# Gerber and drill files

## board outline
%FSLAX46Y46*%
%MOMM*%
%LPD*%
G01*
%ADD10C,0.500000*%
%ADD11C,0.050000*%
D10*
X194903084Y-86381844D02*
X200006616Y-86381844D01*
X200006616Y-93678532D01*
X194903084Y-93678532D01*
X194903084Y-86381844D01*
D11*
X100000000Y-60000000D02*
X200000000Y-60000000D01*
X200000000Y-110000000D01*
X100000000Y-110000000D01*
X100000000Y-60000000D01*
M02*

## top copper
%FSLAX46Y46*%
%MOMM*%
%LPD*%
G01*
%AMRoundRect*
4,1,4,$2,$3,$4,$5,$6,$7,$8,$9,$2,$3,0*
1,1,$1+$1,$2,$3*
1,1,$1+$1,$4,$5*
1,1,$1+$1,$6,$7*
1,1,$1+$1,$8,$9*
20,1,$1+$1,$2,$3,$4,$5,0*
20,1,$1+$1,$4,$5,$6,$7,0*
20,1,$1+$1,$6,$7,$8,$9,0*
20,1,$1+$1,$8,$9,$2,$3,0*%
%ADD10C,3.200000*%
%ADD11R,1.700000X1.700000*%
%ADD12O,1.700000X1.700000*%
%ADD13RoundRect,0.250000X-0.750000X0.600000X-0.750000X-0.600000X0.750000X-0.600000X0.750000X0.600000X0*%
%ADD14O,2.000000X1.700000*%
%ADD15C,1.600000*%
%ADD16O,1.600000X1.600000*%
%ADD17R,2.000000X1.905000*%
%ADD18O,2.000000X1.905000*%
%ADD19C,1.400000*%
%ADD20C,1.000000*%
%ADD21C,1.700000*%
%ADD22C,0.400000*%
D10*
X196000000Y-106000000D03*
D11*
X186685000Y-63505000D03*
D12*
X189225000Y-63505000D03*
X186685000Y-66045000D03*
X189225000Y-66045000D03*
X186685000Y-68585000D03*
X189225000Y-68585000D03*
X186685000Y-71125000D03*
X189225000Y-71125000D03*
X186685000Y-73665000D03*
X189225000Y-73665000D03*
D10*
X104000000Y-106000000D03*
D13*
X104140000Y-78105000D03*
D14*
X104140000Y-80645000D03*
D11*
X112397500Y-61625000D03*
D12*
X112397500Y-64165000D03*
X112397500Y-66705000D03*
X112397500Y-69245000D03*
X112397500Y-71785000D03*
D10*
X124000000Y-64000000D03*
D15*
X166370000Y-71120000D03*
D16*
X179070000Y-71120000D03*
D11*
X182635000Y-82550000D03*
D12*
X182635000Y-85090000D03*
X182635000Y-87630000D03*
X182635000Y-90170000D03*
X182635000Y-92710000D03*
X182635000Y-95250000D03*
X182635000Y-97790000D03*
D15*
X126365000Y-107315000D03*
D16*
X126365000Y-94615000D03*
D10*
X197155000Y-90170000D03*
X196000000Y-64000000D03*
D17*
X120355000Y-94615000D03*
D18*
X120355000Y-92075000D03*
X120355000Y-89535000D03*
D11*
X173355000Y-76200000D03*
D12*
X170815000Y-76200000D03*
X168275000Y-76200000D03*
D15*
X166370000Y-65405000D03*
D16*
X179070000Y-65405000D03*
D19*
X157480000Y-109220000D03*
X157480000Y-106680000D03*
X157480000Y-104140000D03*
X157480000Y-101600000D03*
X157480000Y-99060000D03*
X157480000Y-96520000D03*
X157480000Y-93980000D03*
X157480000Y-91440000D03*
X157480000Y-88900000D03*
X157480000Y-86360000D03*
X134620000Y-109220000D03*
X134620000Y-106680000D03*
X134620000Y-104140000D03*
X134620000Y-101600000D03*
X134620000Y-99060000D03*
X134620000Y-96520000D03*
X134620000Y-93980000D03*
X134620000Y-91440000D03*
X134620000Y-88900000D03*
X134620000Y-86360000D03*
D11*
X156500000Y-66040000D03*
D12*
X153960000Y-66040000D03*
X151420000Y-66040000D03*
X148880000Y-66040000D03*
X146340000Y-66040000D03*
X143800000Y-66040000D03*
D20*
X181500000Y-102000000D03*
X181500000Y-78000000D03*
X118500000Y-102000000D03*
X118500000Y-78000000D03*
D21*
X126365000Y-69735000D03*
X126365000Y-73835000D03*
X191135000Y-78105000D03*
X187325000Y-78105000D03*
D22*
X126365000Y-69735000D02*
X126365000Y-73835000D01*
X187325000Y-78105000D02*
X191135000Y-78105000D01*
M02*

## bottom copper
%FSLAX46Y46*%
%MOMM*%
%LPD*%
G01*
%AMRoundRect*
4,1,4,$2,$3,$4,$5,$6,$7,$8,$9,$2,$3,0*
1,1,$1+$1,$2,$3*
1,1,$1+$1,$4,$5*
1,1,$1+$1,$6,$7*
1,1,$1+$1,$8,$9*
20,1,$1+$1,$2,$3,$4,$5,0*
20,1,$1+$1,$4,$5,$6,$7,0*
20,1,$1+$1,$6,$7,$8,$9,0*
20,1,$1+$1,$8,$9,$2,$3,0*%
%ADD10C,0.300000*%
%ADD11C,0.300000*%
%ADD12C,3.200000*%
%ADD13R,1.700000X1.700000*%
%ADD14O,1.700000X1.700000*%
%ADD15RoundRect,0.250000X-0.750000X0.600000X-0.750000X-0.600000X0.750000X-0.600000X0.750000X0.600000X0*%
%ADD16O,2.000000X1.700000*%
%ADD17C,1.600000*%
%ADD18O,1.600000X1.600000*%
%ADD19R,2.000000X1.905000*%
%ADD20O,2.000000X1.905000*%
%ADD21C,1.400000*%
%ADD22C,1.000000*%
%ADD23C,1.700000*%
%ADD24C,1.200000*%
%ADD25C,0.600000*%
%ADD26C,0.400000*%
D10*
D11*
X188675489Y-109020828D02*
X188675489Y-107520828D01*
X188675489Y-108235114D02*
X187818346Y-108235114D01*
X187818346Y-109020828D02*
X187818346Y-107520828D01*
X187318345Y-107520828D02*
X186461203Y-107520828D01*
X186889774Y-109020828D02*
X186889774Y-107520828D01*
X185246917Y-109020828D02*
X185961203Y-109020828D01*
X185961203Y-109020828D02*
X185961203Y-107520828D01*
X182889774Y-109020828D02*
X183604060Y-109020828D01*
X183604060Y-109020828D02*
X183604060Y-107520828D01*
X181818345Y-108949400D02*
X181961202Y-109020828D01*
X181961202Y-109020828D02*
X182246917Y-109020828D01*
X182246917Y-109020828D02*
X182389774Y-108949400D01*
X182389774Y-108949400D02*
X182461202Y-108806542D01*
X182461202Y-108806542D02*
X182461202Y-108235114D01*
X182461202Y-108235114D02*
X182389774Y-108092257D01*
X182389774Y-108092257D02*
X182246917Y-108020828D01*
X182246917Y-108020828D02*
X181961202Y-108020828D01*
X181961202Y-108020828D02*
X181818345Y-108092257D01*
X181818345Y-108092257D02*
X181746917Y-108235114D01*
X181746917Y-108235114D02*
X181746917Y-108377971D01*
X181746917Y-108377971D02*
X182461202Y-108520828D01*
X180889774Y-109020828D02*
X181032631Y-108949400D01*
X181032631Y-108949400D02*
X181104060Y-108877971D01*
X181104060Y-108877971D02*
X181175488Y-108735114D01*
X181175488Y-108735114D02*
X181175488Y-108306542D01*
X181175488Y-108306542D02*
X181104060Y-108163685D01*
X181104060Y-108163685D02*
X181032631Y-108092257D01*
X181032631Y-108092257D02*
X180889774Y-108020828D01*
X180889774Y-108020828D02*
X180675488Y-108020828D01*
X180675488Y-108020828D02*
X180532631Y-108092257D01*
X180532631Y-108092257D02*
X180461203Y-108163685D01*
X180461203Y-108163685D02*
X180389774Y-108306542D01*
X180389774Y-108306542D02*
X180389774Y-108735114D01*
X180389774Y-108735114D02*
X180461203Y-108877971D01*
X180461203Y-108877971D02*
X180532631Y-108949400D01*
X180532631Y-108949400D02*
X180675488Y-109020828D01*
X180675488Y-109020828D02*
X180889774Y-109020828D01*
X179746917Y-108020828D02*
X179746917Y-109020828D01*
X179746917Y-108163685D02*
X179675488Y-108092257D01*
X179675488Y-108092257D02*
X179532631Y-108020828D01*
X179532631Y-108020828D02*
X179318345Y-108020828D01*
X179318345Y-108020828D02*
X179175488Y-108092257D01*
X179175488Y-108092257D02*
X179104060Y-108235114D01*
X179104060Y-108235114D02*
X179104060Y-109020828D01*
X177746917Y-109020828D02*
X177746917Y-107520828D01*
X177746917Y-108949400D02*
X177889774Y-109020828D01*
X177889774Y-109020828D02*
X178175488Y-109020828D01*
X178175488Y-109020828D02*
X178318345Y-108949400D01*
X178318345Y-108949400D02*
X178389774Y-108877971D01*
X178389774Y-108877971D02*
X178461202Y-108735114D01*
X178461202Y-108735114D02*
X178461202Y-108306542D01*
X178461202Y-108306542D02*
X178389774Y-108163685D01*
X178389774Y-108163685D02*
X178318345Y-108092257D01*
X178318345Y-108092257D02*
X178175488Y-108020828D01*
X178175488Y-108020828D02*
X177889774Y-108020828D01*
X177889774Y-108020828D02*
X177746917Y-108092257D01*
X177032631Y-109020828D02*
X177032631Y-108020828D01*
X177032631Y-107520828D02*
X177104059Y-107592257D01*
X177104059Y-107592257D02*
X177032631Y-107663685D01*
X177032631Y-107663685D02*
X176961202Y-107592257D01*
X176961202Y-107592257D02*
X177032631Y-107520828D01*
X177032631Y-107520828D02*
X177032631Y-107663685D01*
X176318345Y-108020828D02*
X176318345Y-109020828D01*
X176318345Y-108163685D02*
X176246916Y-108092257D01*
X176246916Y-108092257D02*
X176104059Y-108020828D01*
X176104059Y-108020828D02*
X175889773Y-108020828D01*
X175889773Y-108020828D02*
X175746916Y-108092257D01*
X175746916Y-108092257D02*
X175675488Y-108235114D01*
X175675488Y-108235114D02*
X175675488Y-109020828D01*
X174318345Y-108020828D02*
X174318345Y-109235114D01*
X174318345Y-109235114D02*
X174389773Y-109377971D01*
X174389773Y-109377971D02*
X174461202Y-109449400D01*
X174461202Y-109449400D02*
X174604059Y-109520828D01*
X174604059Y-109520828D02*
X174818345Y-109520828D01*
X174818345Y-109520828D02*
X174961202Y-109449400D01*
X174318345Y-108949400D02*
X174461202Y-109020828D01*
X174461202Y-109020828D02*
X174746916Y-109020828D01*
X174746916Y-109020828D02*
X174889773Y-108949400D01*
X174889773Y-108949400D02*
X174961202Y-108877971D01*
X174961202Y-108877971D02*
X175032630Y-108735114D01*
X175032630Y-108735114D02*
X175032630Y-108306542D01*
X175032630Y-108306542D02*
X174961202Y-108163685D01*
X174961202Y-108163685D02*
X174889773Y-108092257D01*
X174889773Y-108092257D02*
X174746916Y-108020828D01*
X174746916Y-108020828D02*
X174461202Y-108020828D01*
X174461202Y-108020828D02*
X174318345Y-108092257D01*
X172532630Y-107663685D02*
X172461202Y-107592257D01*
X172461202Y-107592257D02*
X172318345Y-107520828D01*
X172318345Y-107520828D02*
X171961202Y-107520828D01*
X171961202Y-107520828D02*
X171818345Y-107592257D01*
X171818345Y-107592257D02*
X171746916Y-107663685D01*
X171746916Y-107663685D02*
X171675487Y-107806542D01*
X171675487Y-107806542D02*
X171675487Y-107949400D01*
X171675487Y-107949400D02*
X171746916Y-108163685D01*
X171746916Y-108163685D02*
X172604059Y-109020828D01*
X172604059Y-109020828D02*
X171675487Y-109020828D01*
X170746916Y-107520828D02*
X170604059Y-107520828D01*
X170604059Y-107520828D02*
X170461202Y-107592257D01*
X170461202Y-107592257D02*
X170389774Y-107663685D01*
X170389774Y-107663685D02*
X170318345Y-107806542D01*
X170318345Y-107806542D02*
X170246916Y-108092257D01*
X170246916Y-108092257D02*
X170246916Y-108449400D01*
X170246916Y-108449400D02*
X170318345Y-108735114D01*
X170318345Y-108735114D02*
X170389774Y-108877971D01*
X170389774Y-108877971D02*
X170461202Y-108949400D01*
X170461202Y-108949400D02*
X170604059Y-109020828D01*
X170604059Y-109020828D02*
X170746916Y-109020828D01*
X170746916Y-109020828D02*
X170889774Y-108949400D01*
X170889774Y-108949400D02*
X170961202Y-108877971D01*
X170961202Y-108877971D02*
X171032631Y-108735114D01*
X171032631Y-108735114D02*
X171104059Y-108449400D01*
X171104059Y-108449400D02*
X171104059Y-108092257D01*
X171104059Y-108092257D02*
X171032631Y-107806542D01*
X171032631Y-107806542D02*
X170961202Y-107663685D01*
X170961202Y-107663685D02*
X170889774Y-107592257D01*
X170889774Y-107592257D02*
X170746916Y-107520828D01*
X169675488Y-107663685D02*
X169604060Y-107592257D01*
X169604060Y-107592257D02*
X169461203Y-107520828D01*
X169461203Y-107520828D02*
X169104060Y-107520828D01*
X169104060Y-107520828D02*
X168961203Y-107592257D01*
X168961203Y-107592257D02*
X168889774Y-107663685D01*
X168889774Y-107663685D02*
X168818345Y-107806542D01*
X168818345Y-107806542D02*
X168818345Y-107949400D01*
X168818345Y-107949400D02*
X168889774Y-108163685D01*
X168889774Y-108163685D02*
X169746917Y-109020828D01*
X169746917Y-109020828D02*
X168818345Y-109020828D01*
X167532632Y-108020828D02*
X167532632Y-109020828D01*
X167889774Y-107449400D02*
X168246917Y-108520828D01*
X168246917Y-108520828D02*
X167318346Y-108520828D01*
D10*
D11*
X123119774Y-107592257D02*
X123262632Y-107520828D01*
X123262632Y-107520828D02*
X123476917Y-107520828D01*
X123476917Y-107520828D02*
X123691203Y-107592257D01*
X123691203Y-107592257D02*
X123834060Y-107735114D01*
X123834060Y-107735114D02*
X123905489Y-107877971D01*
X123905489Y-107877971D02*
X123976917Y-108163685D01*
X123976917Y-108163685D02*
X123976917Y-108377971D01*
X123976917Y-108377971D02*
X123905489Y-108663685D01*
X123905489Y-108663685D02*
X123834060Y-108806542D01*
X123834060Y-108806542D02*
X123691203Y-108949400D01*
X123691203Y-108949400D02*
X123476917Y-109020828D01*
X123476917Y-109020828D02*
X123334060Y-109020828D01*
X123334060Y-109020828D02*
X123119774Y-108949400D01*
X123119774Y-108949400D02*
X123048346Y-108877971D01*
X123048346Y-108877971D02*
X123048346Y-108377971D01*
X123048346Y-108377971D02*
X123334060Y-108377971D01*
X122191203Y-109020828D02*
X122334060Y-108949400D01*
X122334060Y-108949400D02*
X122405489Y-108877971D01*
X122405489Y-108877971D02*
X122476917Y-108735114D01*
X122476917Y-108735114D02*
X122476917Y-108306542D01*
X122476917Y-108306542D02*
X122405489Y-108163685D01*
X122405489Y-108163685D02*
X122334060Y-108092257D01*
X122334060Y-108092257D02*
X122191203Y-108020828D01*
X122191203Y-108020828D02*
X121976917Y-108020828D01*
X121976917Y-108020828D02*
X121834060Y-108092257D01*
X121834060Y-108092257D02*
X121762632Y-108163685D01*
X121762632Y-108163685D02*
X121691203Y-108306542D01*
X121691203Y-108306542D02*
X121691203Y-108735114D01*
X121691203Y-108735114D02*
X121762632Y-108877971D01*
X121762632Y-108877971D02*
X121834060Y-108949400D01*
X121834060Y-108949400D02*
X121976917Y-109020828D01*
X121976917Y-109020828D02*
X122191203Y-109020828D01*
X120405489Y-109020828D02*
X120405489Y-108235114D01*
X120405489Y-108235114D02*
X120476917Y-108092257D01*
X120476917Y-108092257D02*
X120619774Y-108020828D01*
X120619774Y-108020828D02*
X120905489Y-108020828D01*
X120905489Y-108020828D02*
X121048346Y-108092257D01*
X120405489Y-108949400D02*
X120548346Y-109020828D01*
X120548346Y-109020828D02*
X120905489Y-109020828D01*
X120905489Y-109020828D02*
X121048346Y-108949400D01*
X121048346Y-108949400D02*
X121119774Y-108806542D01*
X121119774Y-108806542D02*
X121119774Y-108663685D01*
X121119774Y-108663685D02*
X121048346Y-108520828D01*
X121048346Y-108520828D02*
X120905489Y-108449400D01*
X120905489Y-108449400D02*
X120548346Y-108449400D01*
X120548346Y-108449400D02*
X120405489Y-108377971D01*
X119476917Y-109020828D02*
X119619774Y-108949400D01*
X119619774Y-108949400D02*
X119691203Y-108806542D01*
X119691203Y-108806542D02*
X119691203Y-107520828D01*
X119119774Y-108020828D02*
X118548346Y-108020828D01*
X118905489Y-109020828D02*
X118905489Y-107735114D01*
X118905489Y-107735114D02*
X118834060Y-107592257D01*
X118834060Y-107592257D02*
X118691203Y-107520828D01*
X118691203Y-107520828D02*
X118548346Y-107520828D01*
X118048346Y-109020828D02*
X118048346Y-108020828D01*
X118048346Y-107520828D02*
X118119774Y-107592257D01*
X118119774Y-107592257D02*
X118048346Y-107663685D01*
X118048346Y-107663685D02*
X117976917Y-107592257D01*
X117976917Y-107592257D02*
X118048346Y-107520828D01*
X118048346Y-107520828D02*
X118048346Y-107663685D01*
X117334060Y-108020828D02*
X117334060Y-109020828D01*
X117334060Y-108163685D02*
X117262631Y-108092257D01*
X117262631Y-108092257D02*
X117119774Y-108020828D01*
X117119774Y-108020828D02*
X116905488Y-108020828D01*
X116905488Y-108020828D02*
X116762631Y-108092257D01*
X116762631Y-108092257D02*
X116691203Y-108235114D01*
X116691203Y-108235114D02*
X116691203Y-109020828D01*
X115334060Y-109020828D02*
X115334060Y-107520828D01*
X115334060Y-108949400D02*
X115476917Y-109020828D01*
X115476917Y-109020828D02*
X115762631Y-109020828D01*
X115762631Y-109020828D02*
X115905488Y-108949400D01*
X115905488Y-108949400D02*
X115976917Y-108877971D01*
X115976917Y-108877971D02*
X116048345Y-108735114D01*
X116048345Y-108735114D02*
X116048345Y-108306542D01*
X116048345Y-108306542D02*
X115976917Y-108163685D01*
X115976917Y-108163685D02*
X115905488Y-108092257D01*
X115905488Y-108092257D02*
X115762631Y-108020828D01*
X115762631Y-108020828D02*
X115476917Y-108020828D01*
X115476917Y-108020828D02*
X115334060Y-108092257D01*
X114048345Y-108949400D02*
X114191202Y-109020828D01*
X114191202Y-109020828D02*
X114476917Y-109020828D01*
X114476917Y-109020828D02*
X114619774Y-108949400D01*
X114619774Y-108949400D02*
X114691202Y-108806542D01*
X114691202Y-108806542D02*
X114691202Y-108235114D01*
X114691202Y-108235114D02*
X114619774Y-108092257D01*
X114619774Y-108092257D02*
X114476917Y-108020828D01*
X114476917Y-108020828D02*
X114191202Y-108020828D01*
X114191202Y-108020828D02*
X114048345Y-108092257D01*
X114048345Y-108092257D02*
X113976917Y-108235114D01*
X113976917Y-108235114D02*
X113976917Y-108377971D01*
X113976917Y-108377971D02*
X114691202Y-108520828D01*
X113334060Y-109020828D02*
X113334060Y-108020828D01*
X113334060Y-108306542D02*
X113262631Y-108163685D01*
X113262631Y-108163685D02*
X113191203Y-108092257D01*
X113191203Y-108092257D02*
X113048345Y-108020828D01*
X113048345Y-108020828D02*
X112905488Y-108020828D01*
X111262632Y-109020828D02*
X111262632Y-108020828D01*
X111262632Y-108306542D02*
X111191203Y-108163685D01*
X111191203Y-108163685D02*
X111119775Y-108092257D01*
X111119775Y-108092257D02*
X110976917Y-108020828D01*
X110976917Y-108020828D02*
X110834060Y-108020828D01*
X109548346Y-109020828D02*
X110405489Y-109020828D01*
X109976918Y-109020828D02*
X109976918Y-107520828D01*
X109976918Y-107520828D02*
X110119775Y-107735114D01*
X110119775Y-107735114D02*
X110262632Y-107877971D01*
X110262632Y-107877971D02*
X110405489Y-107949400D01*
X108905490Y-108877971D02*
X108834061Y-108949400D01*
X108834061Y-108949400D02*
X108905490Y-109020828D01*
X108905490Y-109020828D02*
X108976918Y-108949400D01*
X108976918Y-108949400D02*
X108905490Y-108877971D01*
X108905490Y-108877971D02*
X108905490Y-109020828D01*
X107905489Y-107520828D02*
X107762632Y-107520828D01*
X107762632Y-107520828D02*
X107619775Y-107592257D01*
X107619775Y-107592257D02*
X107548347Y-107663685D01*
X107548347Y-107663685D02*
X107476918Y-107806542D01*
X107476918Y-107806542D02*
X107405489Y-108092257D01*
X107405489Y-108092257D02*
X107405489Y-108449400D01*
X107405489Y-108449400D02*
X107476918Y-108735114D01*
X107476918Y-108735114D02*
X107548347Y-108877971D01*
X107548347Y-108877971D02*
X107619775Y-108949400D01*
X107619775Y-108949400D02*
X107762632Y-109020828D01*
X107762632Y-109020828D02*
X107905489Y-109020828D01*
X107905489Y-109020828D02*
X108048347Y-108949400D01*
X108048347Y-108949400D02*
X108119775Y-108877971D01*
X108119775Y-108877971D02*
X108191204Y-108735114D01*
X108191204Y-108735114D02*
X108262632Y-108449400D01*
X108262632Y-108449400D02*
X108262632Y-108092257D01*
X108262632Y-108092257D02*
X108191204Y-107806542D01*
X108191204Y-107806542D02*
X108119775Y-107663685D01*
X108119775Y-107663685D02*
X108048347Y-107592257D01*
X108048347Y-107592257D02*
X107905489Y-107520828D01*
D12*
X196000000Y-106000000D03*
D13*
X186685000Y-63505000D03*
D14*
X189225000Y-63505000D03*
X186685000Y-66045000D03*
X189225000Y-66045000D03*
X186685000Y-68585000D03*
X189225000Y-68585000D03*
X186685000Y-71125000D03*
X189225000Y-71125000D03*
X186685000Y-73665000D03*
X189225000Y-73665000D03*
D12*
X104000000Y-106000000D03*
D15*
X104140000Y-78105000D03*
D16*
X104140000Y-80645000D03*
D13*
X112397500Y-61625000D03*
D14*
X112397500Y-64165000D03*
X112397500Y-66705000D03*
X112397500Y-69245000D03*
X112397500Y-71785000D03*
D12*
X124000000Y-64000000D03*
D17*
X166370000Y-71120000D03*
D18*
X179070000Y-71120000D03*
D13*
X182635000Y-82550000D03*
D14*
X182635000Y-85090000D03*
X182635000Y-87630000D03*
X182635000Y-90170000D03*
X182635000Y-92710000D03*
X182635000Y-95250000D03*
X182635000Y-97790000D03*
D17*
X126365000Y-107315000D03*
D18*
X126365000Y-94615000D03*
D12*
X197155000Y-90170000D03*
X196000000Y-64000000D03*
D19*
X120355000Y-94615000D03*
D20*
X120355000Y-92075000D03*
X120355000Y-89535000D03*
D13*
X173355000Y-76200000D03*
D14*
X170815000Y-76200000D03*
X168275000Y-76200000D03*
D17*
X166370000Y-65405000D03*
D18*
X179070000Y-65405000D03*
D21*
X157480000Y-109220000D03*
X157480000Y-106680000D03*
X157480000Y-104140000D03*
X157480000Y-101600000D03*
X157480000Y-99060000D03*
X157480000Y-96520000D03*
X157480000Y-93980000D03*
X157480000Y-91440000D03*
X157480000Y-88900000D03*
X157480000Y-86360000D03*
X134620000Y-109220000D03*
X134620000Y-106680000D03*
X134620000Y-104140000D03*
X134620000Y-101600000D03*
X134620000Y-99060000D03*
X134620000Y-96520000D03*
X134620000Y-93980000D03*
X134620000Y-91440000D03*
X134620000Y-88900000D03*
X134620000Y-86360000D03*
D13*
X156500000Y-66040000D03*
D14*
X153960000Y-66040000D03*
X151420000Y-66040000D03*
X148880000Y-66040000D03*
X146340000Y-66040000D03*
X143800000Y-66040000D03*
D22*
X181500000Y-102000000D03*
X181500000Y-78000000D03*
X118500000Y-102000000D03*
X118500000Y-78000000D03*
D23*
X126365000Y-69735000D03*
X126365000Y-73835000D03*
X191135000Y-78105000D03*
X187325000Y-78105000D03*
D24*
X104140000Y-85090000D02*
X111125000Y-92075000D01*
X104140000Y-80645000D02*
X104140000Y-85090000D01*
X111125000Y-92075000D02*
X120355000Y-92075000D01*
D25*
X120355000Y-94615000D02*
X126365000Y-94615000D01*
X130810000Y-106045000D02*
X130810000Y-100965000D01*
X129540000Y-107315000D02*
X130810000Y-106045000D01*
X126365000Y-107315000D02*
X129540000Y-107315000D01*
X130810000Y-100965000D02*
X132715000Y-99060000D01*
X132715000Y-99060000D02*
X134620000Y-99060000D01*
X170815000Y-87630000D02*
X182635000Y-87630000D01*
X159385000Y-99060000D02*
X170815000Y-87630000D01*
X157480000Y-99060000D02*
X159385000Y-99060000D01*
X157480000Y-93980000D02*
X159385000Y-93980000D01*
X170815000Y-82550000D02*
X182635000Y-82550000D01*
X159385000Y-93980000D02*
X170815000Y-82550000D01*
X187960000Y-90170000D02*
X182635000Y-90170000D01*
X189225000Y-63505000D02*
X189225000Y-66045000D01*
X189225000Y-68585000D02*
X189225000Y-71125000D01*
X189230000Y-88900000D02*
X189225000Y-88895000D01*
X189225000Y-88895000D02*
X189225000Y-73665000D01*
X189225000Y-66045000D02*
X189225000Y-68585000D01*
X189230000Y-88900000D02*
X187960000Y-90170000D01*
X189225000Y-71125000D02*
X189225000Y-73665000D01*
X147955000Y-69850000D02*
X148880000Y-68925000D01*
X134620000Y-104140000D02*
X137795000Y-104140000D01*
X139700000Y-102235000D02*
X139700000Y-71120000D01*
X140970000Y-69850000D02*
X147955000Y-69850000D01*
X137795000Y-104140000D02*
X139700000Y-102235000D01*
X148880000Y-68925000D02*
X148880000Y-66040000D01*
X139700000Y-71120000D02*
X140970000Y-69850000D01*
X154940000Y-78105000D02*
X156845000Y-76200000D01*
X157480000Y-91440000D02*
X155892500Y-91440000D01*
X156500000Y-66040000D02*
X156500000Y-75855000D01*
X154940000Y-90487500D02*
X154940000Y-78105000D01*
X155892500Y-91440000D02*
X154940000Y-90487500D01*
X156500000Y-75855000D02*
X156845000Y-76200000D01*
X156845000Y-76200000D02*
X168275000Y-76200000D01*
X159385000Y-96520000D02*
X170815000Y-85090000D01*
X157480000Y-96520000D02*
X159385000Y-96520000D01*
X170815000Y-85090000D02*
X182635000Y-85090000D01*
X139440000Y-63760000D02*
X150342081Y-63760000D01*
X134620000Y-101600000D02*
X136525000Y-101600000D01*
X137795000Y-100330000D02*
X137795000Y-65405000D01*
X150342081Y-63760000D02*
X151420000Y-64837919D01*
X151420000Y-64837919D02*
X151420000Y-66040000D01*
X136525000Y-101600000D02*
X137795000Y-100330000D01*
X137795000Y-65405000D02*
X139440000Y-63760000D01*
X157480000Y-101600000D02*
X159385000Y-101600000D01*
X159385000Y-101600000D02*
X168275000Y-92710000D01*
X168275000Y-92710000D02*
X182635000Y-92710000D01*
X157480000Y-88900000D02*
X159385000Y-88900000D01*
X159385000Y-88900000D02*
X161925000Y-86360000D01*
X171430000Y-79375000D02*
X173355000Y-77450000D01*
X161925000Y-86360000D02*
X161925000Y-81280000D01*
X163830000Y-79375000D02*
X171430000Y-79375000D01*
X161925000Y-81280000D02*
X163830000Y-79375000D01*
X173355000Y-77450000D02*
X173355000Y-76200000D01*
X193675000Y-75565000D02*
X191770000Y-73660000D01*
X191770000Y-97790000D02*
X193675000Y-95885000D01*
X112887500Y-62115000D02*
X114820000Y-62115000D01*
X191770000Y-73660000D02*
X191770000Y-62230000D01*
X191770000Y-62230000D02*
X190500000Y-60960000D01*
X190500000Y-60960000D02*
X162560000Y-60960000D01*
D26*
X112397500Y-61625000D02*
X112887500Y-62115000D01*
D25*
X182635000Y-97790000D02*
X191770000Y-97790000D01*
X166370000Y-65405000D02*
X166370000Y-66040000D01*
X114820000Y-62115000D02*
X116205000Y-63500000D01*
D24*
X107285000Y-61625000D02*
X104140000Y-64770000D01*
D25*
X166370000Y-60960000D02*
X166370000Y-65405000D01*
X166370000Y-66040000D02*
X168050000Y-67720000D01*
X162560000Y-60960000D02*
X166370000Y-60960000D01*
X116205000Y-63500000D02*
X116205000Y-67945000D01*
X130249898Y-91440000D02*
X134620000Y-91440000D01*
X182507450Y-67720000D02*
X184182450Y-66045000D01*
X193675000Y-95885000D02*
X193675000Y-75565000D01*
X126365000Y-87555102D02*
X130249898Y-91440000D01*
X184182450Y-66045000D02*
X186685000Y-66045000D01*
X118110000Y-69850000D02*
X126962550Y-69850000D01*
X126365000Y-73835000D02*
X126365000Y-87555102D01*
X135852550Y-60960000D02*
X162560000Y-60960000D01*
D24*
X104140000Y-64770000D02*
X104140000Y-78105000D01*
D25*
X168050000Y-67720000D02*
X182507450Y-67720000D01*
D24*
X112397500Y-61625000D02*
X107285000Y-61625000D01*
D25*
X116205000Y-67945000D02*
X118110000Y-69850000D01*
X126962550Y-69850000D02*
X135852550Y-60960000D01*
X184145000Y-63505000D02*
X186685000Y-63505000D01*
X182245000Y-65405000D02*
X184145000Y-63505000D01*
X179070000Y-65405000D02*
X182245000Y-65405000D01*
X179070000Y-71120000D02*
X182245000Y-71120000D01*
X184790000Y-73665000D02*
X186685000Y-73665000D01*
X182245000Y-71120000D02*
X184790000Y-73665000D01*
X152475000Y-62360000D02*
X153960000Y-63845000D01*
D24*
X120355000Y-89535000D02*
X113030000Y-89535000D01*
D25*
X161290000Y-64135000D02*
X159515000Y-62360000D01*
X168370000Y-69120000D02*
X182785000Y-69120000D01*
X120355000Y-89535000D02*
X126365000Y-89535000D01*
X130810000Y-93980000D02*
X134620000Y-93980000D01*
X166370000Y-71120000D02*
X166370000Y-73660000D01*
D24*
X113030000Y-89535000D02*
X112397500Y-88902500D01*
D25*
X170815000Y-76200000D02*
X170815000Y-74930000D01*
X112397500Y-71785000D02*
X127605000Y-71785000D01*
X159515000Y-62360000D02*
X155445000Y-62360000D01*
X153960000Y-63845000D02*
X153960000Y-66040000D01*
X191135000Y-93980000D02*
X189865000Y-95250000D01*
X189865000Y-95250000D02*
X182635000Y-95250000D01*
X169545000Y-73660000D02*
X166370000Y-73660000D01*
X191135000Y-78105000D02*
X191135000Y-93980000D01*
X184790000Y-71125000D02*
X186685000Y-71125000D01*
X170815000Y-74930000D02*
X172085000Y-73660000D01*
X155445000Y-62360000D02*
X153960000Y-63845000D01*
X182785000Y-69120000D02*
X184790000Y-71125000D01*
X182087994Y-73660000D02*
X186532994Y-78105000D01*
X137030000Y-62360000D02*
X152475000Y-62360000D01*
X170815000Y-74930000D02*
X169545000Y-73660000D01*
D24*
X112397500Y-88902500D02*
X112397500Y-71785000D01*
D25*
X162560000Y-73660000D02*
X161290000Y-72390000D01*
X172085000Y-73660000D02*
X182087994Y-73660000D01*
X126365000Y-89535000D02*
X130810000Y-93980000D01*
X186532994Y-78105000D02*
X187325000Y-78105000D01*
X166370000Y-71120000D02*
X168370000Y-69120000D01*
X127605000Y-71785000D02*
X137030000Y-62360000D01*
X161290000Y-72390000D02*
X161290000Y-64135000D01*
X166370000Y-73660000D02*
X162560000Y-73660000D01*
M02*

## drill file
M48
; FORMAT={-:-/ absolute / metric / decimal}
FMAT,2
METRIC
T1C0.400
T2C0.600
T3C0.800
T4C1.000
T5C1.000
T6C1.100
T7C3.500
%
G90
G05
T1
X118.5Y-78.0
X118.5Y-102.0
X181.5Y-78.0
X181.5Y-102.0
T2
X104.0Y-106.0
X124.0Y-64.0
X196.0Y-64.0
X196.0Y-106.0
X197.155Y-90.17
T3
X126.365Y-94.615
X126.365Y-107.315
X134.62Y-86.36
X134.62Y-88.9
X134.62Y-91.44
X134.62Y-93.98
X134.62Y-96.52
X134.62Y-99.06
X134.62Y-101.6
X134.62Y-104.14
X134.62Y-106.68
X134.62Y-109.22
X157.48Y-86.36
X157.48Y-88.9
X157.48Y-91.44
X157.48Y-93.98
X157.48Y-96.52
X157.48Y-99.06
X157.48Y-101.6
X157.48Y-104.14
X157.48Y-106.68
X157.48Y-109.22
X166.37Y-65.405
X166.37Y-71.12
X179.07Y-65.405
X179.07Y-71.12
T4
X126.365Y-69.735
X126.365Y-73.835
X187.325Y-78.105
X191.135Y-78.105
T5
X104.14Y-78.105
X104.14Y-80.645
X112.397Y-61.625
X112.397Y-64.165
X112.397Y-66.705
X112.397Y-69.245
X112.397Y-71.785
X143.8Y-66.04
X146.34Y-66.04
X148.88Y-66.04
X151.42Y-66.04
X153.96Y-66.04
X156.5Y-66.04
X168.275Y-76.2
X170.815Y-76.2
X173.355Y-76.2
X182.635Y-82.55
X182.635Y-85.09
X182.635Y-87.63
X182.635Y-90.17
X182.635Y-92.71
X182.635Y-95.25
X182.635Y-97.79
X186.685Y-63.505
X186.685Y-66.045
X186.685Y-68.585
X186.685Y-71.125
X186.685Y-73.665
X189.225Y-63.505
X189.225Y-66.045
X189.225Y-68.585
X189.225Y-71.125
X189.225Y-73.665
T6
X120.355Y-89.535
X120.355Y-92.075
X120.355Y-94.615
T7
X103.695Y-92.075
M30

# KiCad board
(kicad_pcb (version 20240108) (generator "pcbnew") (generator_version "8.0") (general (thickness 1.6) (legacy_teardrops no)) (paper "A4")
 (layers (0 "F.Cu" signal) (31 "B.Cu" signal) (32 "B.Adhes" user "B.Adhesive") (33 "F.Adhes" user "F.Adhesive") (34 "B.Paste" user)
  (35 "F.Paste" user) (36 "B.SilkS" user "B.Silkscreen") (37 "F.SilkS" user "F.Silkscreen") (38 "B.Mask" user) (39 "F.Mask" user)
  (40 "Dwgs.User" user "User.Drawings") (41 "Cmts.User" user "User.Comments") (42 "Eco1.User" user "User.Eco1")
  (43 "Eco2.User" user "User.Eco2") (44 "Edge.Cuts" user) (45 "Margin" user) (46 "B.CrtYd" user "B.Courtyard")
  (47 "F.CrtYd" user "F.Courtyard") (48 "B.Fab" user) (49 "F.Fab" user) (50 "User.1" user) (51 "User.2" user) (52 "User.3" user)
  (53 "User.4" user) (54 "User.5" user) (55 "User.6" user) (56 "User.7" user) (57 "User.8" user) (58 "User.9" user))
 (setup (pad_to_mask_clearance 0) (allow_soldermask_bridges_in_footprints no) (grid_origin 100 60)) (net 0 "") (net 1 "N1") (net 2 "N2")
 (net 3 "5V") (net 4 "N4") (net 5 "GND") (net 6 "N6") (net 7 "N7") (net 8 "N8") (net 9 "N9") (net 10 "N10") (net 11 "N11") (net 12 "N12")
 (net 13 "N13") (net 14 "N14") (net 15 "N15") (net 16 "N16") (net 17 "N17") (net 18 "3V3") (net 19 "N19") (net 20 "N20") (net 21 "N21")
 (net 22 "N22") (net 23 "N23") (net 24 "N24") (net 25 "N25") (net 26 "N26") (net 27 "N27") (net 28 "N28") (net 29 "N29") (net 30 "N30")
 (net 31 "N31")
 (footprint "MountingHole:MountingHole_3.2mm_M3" (layer "F.Cu") (at 196 106 -90)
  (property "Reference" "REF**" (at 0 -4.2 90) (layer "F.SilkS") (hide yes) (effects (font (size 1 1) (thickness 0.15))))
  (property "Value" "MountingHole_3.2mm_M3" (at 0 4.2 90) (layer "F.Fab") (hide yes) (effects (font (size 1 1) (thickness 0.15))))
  (pad "" thru_hole circle (at 0 0 270) (size 3.2 3.2) (drill 0.6) (layers "*.Cu" "*.Mask") (remove_unused_layers no)))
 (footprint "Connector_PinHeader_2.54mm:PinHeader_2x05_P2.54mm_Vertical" (layer "F.Cu") (at 186.685 63.505)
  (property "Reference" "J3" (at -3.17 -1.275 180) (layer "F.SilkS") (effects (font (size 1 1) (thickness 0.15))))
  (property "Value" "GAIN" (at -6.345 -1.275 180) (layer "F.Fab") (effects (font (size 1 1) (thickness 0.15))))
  (pad "1" thru_hole rect (at 0 0) (size 1.7 1.7) (drill 1) (layers "*.Cu" "*.Mask") (remove_unused_layers no) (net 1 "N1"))
  (pad "2" thru_hole oval (at 2.54 0) (size 1.7 1.7) (drill 1) (layers "*.Cu" "*.Mask") (remove_unused_layers no) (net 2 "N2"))
  (pad "3" thru_hole oval (at 0 2.54) (size 1.7 1.7) (drill 1) (layers "*.Cu" "*.Mask") (remove_unused_layers no) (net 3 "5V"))
  (pad "4" thru_hole oval (at 2.54 2.54) (size 1.7 1.7) (drill 1) (layers "*.Cu" "*.Mask") (remove_unused_layers no) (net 2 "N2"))
  (pad "5" thru_hole oval (at 0 5.08) (size 1.7 1.7) (drill 1) (layers "*.Cu" "*.Mask") (remove_unused_layers no) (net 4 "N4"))
  (pad "6" thru_hole oval (at 2.54 5.08) (size 1.7 1.7) (drill 1) (layers "*.Cu" "*.Mask") (remove_unused_layers no) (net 2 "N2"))
  (pad "7" thru_hole oval (at 0 7.62) (size 1.7 1.7) (drill 1) (layers "*.Cu" "*.Mask") (remove_unused_layers no) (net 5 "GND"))
  (pad "8" thru_hole oval (at 2.54 7.62) (size 1.7 1.7) (drill 1) (layers "*.Cu" "*.Mask") (remove_unused_layers no) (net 2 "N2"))
  (pad "9" thru_hole oval (at 0 10.16) (size 1.7 1.7) (drill 1) (layers "*.Cu" "*.Mask") (remove_unused_layers no) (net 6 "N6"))
  (pad "10" thru_hole oval (at 2.54 10.16) (size 1.7 1.7) (drill 1) (layers "*.Cu" "*.Mask") (remove_unused_layers no) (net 2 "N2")))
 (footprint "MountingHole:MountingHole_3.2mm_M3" (layer "F.Cu") (at 104 106 -90)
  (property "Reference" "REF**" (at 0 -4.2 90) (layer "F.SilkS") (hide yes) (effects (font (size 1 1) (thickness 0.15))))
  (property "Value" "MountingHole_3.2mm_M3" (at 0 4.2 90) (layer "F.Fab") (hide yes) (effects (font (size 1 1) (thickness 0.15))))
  (pad "" thru_hole circle (at 0 0 270) (size 3.2 3.2) (drill 0.6) (layers "*.Cu" "*.Mask") (remove_unused_layers no)))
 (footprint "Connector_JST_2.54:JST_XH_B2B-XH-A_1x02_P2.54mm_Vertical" (layer "F.Cu") (at 104.14 78.105 -90)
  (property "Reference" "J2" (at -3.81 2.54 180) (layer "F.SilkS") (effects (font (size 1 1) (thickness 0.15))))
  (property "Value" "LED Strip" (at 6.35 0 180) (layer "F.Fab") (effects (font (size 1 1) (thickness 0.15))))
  (pad "1" thru_hole roundrect (at 0 0 270) (size 1.7 2) (drill 1) (layers "*.Cu" "*.Mask") (remove_unused_layers no)
   (roundrect_rratio 0.147059) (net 3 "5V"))
  (pad "2" thru_hole oval (at 2.54 0 270) (size 1.7 2) (drill 1) (layers "*.Cu" "*.Mask") (remove_unused_layers no) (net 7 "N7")))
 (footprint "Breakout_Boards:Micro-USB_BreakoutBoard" (layer "F.Cu") (at 112.3975 61.625)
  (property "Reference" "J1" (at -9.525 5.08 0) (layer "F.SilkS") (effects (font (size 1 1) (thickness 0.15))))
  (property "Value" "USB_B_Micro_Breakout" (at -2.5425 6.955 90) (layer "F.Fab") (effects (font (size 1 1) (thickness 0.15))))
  (pad "1" thru_hole rect (at 0 0) (size 1.7 1.7) (drill 1) (layers "*.Cu" "*.Mask") (remove_unused_layers no) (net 3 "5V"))
  (pad "2" thru_hole oval (at 0 2.54) (size 1.7 1.7) (drill 1) (layers "*.Cu" "*.Mask") (remove_unused_layers no) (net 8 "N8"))
  (pad "3" thru_hole oval (at 0 5.08) (size 1.7 1.7) (drill 1) (layers "*.Cu" "*.Mask") (remove_unused_layers no) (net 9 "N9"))
  (pad "4" thru_hole oval (at 0 7.62) (size 1.7 1.7) (drill 1) (layers "*.Cu" "*.Mask") (remove_unused_layers no) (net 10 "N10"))
  (pad "5" thru_hole oval (at 0 10.16) (size 1.7 1.7) (drill 1) (layers "*.Cu" "*.Mask") (remove_unused_layers no) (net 5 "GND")))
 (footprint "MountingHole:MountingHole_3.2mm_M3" (layer "F.Cu") (at 124 64 -90)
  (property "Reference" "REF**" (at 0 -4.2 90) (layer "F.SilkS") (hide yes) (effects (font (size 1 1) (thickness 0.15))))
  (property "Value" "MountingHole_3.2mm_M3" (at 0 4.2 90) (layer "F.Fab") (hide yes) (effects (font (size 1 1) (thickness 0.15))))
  (pad "" thru_hole circle (at 0 0 270) (size 3.2 3.2) (drill 0.6) (layers "*.Cu" "*.Mask") (remove_unused_layers no)))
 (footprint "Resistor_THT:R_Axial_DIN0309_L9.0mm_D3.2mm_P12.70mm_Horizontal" (layer "F.Cu") (at 166.37 71.12)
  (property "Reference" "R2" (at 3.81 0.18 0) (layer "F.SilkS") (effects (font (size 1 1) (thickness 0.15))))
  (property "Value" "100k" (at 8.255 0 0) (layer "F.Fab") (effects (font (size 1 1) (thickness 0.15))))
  (pad "1" thru_hole circle (at 0 0) (size 1.6 1.6) (drill 0.8) (layers "*.Cu" "*.Mask") (remove_unused_layers no) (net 5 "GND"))
  (pad "2" thru_hole oval (at 12.7 0) (size 1.6 1.6) (drill 0.8) (layers "*.Cu" "*.Mask") (remove_unused_layers no) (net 6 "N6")))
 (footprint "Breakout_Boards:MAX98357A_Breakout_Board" (layer "F.Cu") (at 182.635 82.55)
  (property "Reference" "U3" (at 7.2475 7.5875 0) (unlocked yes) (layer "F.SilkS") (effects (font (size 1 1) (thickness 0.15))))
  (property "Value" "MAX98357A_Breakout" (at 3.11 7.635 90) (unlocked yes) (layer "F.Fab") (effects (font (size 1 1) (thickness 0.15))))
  (pad "1" thru_hole rect (at 0 0) (size 1.7 1.7) (drill 1) (layers "*.Cu" "*.Mask") (remove_unused_layers no) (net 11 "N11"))
  (pad "2" thru_hole oval (at 0 2.54) (size 1.7 1.7) (drill 1) (layers "*.Cu" "*.Mask") (remove_unused_layers no) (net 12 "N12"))
  (pad "3" thru_hole oval (at 0 5.08) (size 1.7 1.7) (drill 1) (layers "*.Cu" "*.Mask") (remove_unused_layers no) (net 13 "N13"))
  (pad "4" thru_hole oval (at 0 7.62) (size 1.7 1.7) (drill 1) (layers "*.Cu" "*.Mask") (remove_unused_layers no) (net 2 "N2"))
  (pad "5" thru_hole oval (at 0 10.16) (size 1.7 1.7) (drill 1) (layers "*.Cu" "*.Mask") (remove_unused_layers no) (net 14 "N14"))
  (pad "6" thru_hole oval (at 0 12.7) (size 1.7 1.7) (drill 1) (layers "*.Cu" "*.Mask") (remove_unused_layers no) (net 5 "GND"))
  (pad "7" thru_hole oval (at 0 15.24) (size 1.7 1.7) (drill 1) (layers "*.Cu" "*.Mask") (remove_unused_layers no) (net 3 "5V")))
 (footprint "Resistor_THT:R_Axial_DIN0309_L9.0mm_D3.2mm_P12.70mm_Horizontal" (layer "F.Cu") (at 126.365 107.315 90)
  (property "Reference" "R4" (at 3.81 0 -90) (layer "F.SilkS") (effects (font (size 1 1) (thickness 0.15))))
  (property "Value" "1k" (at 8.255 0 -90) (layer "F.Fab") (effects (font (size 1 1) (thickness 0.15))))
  (pad "1" thru_hole circle (at 0 0 90) (size 1.6 1.6) (drill 0.8) (layers "*.Cu" "*.Mask") (remove_unused_layers no) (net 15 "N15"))
  (pad "2" thru_hole oval (at 12.7 0 90) (size 1.6 1.6) (drill 0.8) (layers "*.Cu" "*.Mask") (remove_unused_layers no) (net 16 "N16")))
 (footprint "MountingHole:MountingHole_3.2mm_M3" (layer "F.Cu") (at 197.155 90.17 -90)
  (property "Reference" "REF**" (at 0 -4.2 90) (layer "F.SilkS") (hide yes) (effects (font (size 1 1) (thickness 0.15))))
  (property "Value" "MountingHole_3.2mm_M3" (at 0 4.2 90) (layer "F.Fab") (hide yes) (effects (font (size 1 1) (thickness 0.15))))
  (pad "" thru_hole circle (at 0 0 270) (size 3.2 3.2) (drill 0.6) (layers "*.Cu" "*.Mask") (remove_unused_layers no)))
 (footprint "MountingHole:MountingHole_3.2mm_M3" (layer "F.Cu") (at 196 64 -90)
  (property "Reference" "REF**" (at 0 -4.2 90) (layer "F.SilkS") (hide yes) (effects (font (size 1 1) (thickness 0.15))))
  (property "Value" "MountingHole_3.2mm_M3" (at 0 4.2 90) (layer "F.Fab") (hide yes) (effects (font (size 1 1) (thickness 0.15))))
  (pad "" thru_hole circle (at 0 0 270) (size 3.2 3.2) (drill 0.6) (layers "*.Cu" "*.Mask") (remove_unused_layers no)))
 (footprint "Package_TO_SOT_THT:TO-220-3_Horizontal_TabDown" (layer "F.Cu") (at 120.355 94.615 90)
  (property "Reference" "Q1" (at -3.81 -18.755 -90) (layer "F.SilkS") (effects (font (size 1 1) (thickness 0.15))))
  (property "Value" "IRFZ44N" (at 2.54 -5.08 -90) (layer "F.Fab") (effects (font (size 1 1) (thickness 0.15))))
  (pad "" np_thru_hole oval (at 2.54 -16.66 90) (size 3.5 3.5) (drill 3.5) (layers "*.Cu" "*.Mask"))
  (pad "1" thru_hole rect (at 0 0 90) (size 1.905 2) (drill 1.1) (layers "*.Cu" "*.Mask") (remove_unused_layers no) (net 16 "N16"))
  (pad "2" thru_hole oval (at 2.54 0 90) (size 1.905 2) (drill 1.1) (layers "*.Cu" "*.Mask") (remove_unused_layers no) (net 7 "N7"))
  (pad "3" thru_hole oval (at 5.08 0 90) (size 1.905 2) (drill 1.1) (layers "*.Cu" "*.Mask") (remove_unused_layers no) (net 5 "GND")))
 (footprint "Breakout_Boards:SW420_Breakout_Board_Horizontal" (layer "F.Cu") (at 173.355 76.2 -90)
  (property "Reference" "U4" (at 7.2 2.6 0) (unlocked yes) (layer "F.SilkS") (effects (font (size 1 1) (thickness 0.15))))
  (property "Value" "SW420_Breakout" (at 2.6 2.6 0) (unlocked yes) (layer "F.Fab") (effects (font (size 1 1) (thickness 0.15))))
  (pad "1" thru_hole rect (at 0 0 270) (size 1.7 1.7) (drill 1) (layers "*.Cu" "*.Mask") (remove_unused_layers no) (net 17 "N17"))
  (pad "2" thru_hole oval (at 0 2.54 270) (size 1.7 1.7) (drill 1) (layers "*.Cu" "*.Mask") (remove_unused_layers no) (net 5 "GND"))
  (pad "3" thru_hole oval (at 0 5.08 270) (size 1.7 1.7) (drill 1) (layers "*.Cu" "*.Mask") (remove_unused_layers no) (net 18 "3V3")))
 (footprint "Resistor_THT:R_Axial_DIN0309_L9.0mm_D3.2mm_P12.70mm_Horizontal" (layer "F.Cu") (at 166.37 65.405)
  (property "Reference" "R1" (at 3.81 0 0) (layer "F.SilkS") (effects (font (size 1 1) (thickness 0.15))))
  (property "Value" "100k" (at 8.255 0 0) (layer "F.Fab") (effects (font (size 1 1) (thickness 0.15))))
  (pad "1" thru_hole circle (at 0 0) (size 1.6 1.6) (drill 0.8) (layers "*.Cu" "*.Mask") (remove_unused_layers no) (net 3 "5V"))
  (pad "2" thru_hole oval (at 12.7 0) (size 1.6 1.6) (drill 0.8) (layers "*.Cu" "*.Mask") (remove_unused_layers no) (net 1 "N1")))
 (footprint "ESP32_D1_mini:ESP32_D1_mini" (layer "F.Cu") (at 146.05 97.79 180)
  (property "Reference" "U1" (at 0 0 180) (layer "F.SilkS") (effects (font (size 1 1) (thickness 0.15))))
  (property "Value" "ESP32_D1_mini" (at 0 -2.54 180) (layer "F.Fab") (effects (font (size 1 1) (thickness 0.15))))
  (pad "2" thru_hole circle (at -11.43 -11.43 90) (size 1.4 1.4) (drill 0.8) (layers "*.Cu" "*.Mask") (remove_unused_layers no)
   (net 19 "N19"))
  (pad "4" thru_hole circle (at -11.43 -8.89 90) (size 1.4 1.4) (drill 0.8) (layers "*.Cu" "*.Mask") (remove_unused_layers no)
   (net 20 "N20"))
  (pad "6" thru_hole circle (at -11.43 -6.35 90) (size 1.4 1.4) (drill 0.8) (layers "*.Cu" "*.Mask") (remove_unused_layers no)
   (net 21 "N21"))
  (pad "8" thru_hole circle (at -11.43 -3.81 90) (size 1.4 1.4) (drill 0.8) (layers "*.Cu" "*.Mask") (remove_unused_layers no)
   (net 14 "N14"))
  (pad "10" thru_hole circle (at -11.43 -1.27 90) (size 1.4 1.4) (drill 0.8) (layers "*.Cu" "*.Mask") (remove_unused_layers no)
   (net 13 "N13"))
  (pad "12" thru_hole circle (at -11.43 1.27 90) (size 1.4 1.4) (drill 0.8) (layers "*.Cu" "*.Mask") (remove_unused_layers no)
   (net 12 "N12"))
  (pad "14" thru_hole circle (at -11.43 3.81 90) (size 1.4 1.4) (drill 0.8) (layers "*.Cu" "*.Mask") (remove_unused_layers no)
   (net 11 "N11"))
  (pad "16" thru_hole circle (at -11.43 6.35 90) (size 1.4 1.4) (drill 0.8) (layers "*.Cu" "*.Mask") (remove_unused_layers no)
   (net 18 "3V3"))
  (pad "18" thru_hole circle (at -11.43 8.89 90) (size 1.4 1.4) (drill 0.8) (layers "*.Cu" "*.Mask") (remove_unused_layers no)
   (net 17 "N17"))
  (pad "20" thru_hole circle (at -11.43 11.43 90) (size 1.4 1.4) (drill 0.8) (layers "*.Cu" "*.Mask") (remove_unused_layers no)
   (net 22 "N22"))
  (pad "21" thru_hole circle (at 11.43 -11.43 90) (size 1.4 1.4) (drill 0.8) (layers "*.Cu" "*.Mask") (remove_unused_layers no)
   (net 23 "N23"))
  (pad "23" thru_hole circle (at 11.43 -8.89 90) (size 1.4 1.4) (drill 0.8) (layers "*.Cu" "*.Mask") (remove_unused_layers no)
   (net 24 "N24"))
  (pad "25" thru_hole circle (at 11.43 -6.35 90) (size 1.4 1.4) (drill 0.8) (layers "*.Cu" "*.Mask") (remove_unused_layers no)
   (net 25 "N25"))
  (pad "27" thru_hole circle (at 11.43 -3.81 90) (size 1.4 1.4) (drill 0.8) (layers "*.Cu" "*.Mask") (remove_unused_layers no)
   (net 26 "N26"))
  (pad "29" thru_hole circle (at 11.43 -1.27 90) (size 1.4 1.4) (drill 0.8) (layers "*.Cu" "*.Mask") (remove_unused_layers no)
   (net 15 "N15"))
  (pad "31" thru_hole circle (at 11.43 1.27 90) (size 1.4 1.4) (drill 0.8) (layers "*.Cu" "*.Mask") (remove_unused_layers no) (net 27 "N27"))
  (pad "33" thru_hole circle (at 11.43 3.81 90) (size 1.4 1.4) (drill 0.8) (layers "*.Cu" "*.Mask") (remove_unused_layers no) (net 5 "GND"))
  (pad "35" thru_hole circle (at 11.43 6.35 90) (size 1.4 1.4) (drill 0.8) (layers "*.Cu" "*.Mask") (remove_unused_layers no) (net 3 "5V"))
  (pad "37" thru_hole circle (at 11.43 8.89 90) (size 1.4 1.4) (drill 0.8) (layers "*.Cu" "*.Mask") (remove_unused_layers no) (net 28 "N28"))
  (pad "39" thru_hole circle (at 11.43 11.43 90) (size 1.4 1.4) (drill 0.8) (layers "*.Cu" "*.Mask") (remove_unused_layers no)
   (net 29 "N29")))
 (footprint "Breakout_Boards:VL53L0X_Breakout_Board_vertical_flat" (layer "B.Cu") (at 156.5 66.04 90)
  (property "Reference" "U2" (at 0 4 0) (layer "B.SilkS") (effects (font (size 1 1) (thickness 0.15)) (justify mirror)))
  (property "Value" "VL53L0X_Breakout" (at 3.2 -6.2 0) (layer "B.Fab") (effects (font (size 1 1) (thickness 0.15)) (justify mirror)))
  (pad "1" thru_hole rect (at 0 0 90) (size 1.7 1.7) (drill 1) (layers "*.Cu" "*.Mask") (remove_unused_layers no) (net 18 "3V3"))
  (pad "2" thru_hole oval (at 0 -2.54 90) (size 1.7 1.7) (drill 1) (layers "*.Cu" "*.Mask") (remove_unused_layers no) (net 5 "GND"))
  (pad "3" thru_hole oval (at 0 -5.08 90) (size 1.7 1.7) (drill 1) (layers "*.Cu" "*.Mask") (remove_unused_layers no) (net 26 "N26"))
  (pad "4" thru_hole oval (at 0 -7.62 90) (size 1.7 1.7) (drill 1) (layers "*.Cu" "*.Mask") (remove_unused_layers no) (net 25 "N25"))
  (pad "5" thru_hole oval (at 0 -10.16 90) (size 1.7 1.7) (drill 1) (layers "*.Cu" "*.Mask") (remove_unused_layers no) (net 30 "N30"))
  (pad "6" thru_hole oval (at 0 -12.7 90) (size 1.7 1.7) (drill 1) (layers "*.Cu" "*.Mask") (remove_unused_layers no) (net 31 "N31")))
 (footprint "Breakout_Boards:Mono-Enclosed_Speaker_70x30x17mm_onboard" (layer "B.Cu") (at 185 75 180)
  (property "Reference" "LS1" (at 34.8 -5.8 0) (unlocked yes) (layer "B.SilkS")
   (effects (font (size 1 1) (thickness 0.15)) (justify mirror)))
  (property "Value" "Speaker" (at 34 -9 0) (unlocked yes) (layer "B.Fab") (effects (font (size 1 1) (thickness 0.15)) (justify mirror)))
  (pad "" thru_hole circle (at 3.5 -27 180) (size 1 1) (drill 0.4) (layers "*.Cu" "*.Mask") (remove_unused_layers no)
   (teardrops (best_length_ratio 0.5) (max_length 1) (best_width_ratio 1) (max_width 2) (curve_points 0) (filter_ratio 0.9) (enabled no)
    (allow_two_segments no) (prefer_zone_connections no)))
  (pad "" thru_hole circle (at 3.5 -3 180) (size 1 1) (drill 0.4) (layers "*.Cu" "*.Mask") (remove_unused_layers no)
   (teardrops (best_length_ratio 0.5) (max_length 1) (best_width_ratio 1) (max_width 2) (curve_points 0) (filter_ratio 0.9) (enabled no)
    (allow_two_segments no) (prefer_zone_connections no)))
  (pad "" thru_hole circle (at 66.5 -27 180) (size 1 1) (drill 0.4) (layers "*.Cu" "*.Mask") (remove_unused_layers no)
   (teardrops (best_length_ratio 0.5) (max_length 1) (best_width_ratio 1) (max_width 2) (curve_points 0) (filter_ratio 0.9) (enabled no)
    (allow_two_segments no) (prefer_zone_connections no)))
  (pad "" thru_hole circle (at 66.5 -3 180) (size 1 1) (drill 0.4) (layers "*.Cu" "*.Mask") (remove_unused_layers no)
   (teardrops (best_length_ratio 0.5) (max_length 1) (best_width_ratio 1) (max_width 2) (curve_points 0) (filter_ratio 0.9) (enabled no)
    (allow_two_segments no) (prefer_zone_connections no))))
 (gr_rect (start 194.903084 86.381844) (end 200.006616 93.678532) (stroke (width 0.5) (type default)) (fill none) (layer "Edge.Cuts"))
 (gr_rect (start 100 60) (end 200 110) (stroke (width 0.05) (type default)) (fill none) (layer "Edge.Cuts"))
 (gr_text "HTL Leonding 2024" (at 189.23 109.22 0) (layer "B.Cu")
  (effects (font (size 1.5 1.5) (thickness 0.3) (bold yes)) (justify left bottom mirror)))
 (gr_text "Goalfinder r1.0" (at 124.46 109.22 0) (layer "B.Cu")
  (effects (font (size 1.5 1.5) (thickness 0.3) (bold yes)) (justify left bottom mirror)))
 (segment (start 104.14 85.09) (end 111.125 92.075) (width 1.2) (layer "B.Cu") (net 7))
 (segment (start 104.14 80.645) (end 104.14 85.09) (width 1.2) (layer "B.Cu") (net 7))
 (segment (start 111.125 92.075) (end 120.355 92.075) (width 1.2) (layer "B.Cu") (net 7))
 (segment (start 120.355 94.615) (end 126.365 94.615) (width 0.6) (layer "B.Cu") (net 16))
 (segment (start 130.81 106.045) (end 130.81 100.965) (width 0.6) (layer "B.Cu") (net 15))
 (segment (start 129.54 107.315) (end 130.81 106.045) (width 0.6) (layer "B.Cu") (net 15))
 (segment (start 126.365 107.315) (end 129.54 107.315) (width 0.6) (layer "B.Cu") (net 15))
 (segment (start 130.81 100.965) (end 132.715 99.06) (width 0.6) (layer "B.Cu") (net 15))
 (segment (start 132.715 99.06) (end 134.62 99.06) (width 0.6) (layer "B.Cu") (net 15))
 (segment (start 170.815 87.63) (end 182.635 87.63) (width 0.6) (layer "B.Cu") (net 13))
 (segment (start 159.385 99.06) (end 170.815 87.63) (width 0.6) (layer "B.Cu") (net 13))
 (segment (start 157.48 99.06) (end 159.385 99.06) (width 0.6) (layer "B.Cu") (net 13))
 (segment (start 157.48 93.98) (end 159.385 93.98) (width 0.6) (layer "B.Cu") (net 11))
 (segment (start 170.815 82.55) (end 182.635 82.55) (width 0.6) (layer "B.Cu") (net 11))
 (segment (start 159.385 93.98) (end 170.815 82.55) (width 0.6) (layer "B.Cu") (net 11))
 (segment (start 187.96 90.17) (end 182.635 90.17) (width 0.6) (layer "B.Cu") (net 2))
 (segment (start 189.225 63.505) (end 189.225 66.045) (width 0.6) (layer "B.Cu") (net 2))
 (segment (start 189.225 68.585) (end 189.225 71.125) (width 0.6) (layer "B.Cu") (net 2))
 (segment (start 189.23 88.9) (end 189.225 88.895) (width 0.6) (layer "B.Cu") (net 2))
 (segment (start 189.225 88.895) (end 189.225 73.665) (width 0.6) (layer "B.Cu") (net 2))
 (segment (start 189.225 66.045) (end 189.225 68.585) (width 0.6) (layer "B.Cu") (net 2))
 (segment (start 189.23 88.9) (end 187.96 90.17) (width 0.6) (layer "B.Cu") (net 2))
 (segment (start 189.225 71.125) (end 189.225 73.665) (width 0.6) (layer "B.Cu") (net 2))
 (segment (start 147.955 69.85) (end 148.88 68.925) (width 0.6) (layer "B.Cu") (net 25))
 (segment (start 134.62 104.14) (end 137.795 104.14) (width 0.6) (layer "B.Cu") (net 25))
 (segment (start 139.7 102.235) (end 139.7 71.12) (width 0.6) (layer "B.Cu") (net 25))
 (segment (start 140.97 69.85) (end 147.955 69.85) (width 0.6) (layer "B.Cu") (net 25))
 (segment (start 137.795 104.14) (end 139.7 102.235) (width 0.6) (layer "B.Cu") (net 25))
 (segment (start 148.88 68.925) (end 148.88 66.04) (width 0.6) (layer "B.Cu") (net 25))
 (segment (start 139.7 71.12) (end 140.97 69.85) (width 0.6) (layer "B.Cu") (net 25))
 (segment (start 154.94 78.105) (end 156.845 76.2) (width 0.6) (layer "B.Cu") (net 18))
 (segment (start 157.48 91.44) (end 155.8925 91.44) (width 0.6) (layer "B.Cu") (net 18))
 (segment (start 156.5 66.04) (end 156.5 75.855) (width 0.6) (layer "B.Cu") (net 18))
 (segment (start 154.94 90.4875) (end 154.94 78.105) (width 0.6) (layer "B.Cu") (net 18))
 (segment (start 155.8925 91.44) (end 154.94 90.4875) (width 0.6) (layer "B.Cu") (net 18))
 (segment (start 156.5 75.855) (end 156.845 76.2) (width 0.6) (layer "B.Cu") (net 18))
 (segment (start 156.845 76.2) (end 168.275 76.2) (width 0.6) (layer "B.Cu") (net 18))
 (segment (start 159.385 96.52) (end 170.815 85.09) (width 0.6) (layer "B.Cu") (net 12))
 (segment (start 157.48 96.52) (end 159.385 96.52) (width 0.6) (layer "B.Cu") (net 12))
 (segment (start 170.815 85.09) (end 182.635 85.09) (width 0.6) (layer "B.Cu") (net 12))
 (segment (start 139.44 63.76) (end 150.342081 63.76) (width 0.6) (layer "B.Cu") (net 26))
 (segment (start 134.62 101.6) (end 136.525 101.6) (width 0.6) (layer "B.Cu") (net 26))
 (segment (start 137.795 100.33) (end 137.795 65.405) (width 0.6) (layer "B.Cu") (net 26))
 (segment (start 150.342081 63.76) (end 151.42 64.837919) (width 0.6) (layer "B.Cu") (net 26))
 (segment (start 151.42 64.837919) (end 151.42 66.04) (width 0.6) (layer "B.Cu") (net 26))
 (segment (start 136.525 101.6) (end 137.795 100.33) (width 0.6) (layer "B.Cu") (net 26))
 (segment (start 137.795 65.405) (end 139.44 63.76) (width 0.6) (layer "B.Cu") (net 26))
 (segment (start 157.48 101.6) (end 159.385 101.6) (width 0.6) (layer "B.Cu") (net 14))
 (segment (start 159.385 101.6) (end 168.275 92.71) (width 0.6) (layer "B.Cu") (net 14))
 (segment (start 168.275 92.71) (end 182.635 92.71) (width 0.6) (layer "B.Cu") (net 14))
 (segment (start 157.48 88.9) (end 159.385 88.9) (width 0.6) (layer "B.Cu") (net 17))
 (segment (start 159.385 88.9) (end 161.925 86.36) (width 0.6) (layer "B.Cu") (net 17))
 (segment (start 171.43 79.375) (end 173.355 77.45) (width 0.6) (layer "B.Cu") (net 17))
 (segment (start 161.925 86.36) (end 161.925 81.28) (width 0.6) (layer "B.Cu") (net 17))
 (segment (start 163.83 79.375) (end 171.43 79.375) (width 0.6) (layer "B.Cu") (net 17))
 (segment (start 161.925 81.28) (end 163.83 79.375) (width 0.6) (layer "B.Cu") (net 17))
 (segment (start 173.355 77.45) (end 173.355 76.2) (width 0.6) (layer "B.Cu") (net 17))
 (segment (start 126.365 69.735) (end 126.365 73.835) (width 0.4) (layer "F.Cu") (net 3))
 (via (at 126.365 69.735) (size 1.7) (drill 1) (layers "F.Cu" "B.Cu") (free yes) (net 3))
 (via (at 126.365 73.835) (size 1.7) (drill 1) (layers "F.Cu" "B.Cu") (free yes) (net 3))
 (segment (start 193.675 75.565) (end 191.77 73.66) (width 0.6) (layer "B.Cu") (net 3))
 (segment (start 191.77 97.79) (end 193.675 95.885) (width 0.6) (layer "B.Cu") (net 3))
 (segment (start 112.8875 62.115) (end 114.82 62.115) (width 0.6) (layer "B.Cu") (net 3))
 (segment (start 191.77 73.66) (end 191.77 62.23) (width 0.6) (layer "B.Cu") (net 3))
 (segment (start 191.77 62.23) (end 190.5 60.96) (width 0.6) (layer "B.Cu") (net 3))
 (segment (start 190.5 60.96) (end 162.56 60.96) (width 0.6) (layer "B.Cu") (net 3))
 (segment (start 112.3975 61.625) (end 112.8875 62.115) (width 0.4) (layer "B.Cu") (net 3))
 (segment (start 182.635 97.79) (end 191.77 97.79) (width 0.6) (layer "B.Cu") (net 3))
 (segment (start 166.37 65.405) (end 166.37 66.04) (width 0.6) (layer "B.Cu") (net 3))
 (segment (start 114.82 62.115) (end 116.205 63.5) (width 0.6) (layer "B.Cu") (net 3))
 (segment (start 107.285 61.625) (end 104.14 64.77) (width 1.2) (layer "B.Cu") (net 3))
 (segment (start 166.37 60.96) (end 166.37 65.405) (width 0.6) (layer "B.Cu") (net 3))
 (segment (start 166.37 66.04) (end 168.05 67.72) (width 0.6) (layer "B.Cu") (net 3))
 (segment (start 162.56 60.96) (end 166.37 60.96) (width 0.6) (layer "B.Cu") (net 3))
 (segment (start 116.205 63.5) (end 116.205 67.945) (width 0.6) (layer "B.Cu") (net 3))
 (segment (start 130.249898 91.44) (end 134.62 91.44) (width 0.6) (layer "B.Cu") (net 3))
 (segment (start 182.50745 67.72) (end 184.18245 66.045) (width 0.6) (layer "B.Cu") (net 3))
 (segment (start 193.675 95.885) (end 193.675 75.565) (width 0.6) (layer "B.Cu") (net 3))
 (segment (start 126.365 87.555102) (end 130.249898 91.44) (width 0.6) (layer "B.Cu") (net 3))
 (segment (start 184.18245 66.045) (end 186.685 66.045) (width 0.6) (layer "B.Cu") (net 3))
 (segment (start 118.11 69.85) (end 126.96255 69.85) (width 0.6) (layer "B.Cu") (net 3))
 (segment (start 126.365 73.835) (end 126.365 87.555102) (width 0.6) (layer "B.Cu") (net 3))
 (segment (start 135.85255 60.96) (end 162.56 60.96) (width 0.6) (layer "B.Cu") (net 3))
 (segment (start 104.14 64.77) (end 104.14 78.105) (width 1.2) (layer "B.Cu") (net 3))
 (segment (start 168.05 67.72) (end 182.50745 67.72) (width 0.6) (layer "B.Cu") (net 3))
 (segment (start 112.3975 61.625) (end 107.285 61.625) (width 1.2) (layer "B.Cu") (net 3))
 (segment (start 116.205 67.945) (end 118.11 69.85) (width 0.6) (layer "B.Cu") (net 3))
 (segment (start 126.96255 69.85) (end 135.85255 60.96) (width 0.6) (layer "B.Cu") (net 3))
 (segment (start 184.145 63.505) (end 186.685 63.505) (width 0.6) (layer "B.Cu") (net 1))
 (segment (start 182.245 65.405) (end 184.145 63.505) (width 0.6) (layer "B.Cu") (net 1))
 (segment (start 179.07 65.405) (end 182.245 65.405) (width 0.6) (layer "B.Cu") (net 1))
 (segment (start 179.07 71.12) (end 182.245 71.12) (width 0.6) (layer "B.Cu") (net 6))
 (segment (start 184.79 73.665) (end 186.685 73.665) (width 0.6) (layer "B.Cu") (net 6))
 (segment (start 182.245 71.12) (end 184.79 73.665) (width 0.6) (layer "B.Cu") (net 6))
 (segment (start 187.325 78.105) (end 191.135 78.105) (width 0.4) (layer "F.Cu") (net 5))
 (via (at 191.135 78.105) (size 1.7) (drill 1) (layers "F.Cu" "B.Cu") (free yes) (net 5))
 (via (at 187.325 78.105) (size 1.7) (drill 1) (layers "F.Cu" "B.Cu") (free yes) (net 5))
 (segment (start 152.475 62.36) (end 153.96 63.845) (width 0.6) (layer "B.Cu") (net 5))
 (segment (start 120.355 89.535) (end 113.03 89.535) (width 1.2) (layer "B.Cu") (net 5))
 (segment (start 161.29 64.135) (end 159.515 62.36) (width 0.6) (layer "B.Cu") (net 5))
 (segment (start 168.37 69.12) (end 182.785 69.12) (width 0.6) (layer "B.Cu") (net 5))
 (segment (start 120.355 89.535) (end 126.365 89.535) (width 0.6) (layer "B.Cu") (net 5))
 (segment (start 130.81 93.98) (end 134.62 93.98) (width 0.6) (layer "B.Cu") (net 5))
 (segment (start 166.37 71.12) (end 166.37 73.66) (width 0.6) (layer "B.Cu") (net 5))
 (segment (start 113.03 89.535) (end 112.3975 88.9025) (width 1.2) (layer "B.Cu") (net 5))
 (segment (start 170.815 76.2) (end 170.815 74.93) (width 0.6) (layer "B.Cu") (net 5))
 (segment (start 112.3975 71.785) (end 127.605 71.785) (width 0.6) (layer "B.Cu") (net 5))
 (segment (start 159.515 62.36) (end 155.445 62.36) (width 0.6) (layer "B.Cu") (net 5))
 (segment (start 153.96 63.845) (end 153.96 66.04) (width 0.6) (layer "B.Cu") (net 5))
 (segment (start 191.135 93.98) (end 189.865 95.25) (width 0.6) (layer "B.Cu") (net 5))
 (segment (start 189.865 95.25) (end 182.635 95.25) (width 0.6) (layer "B.Cu") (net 5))
 (segment (start 169.545 73.66) (end 166.37 73.66) (width 0.6) (layer "B.Cu") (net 5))
 (segment (start 191.135 78.105) (end 191.135 93.98) (width 0.6) (layer "B.Cu") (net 5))
 (segment (start 184.79 71.125) (end 186.685 71.125) (width 0.6) (layer "B.Cu") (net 5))
 (segment (start 170.815 74.93) (end 172.085 73.66) (width 0.6) (layer "B.Cu") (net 5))
 (segment (start 155.445 62.36) (end 153.96 63.845) (width 0.6) (layer "B.Cu") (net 5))
 (segment (start 182.785 69.12) (end 184.79 71.125) (width 0.6) (layer "B.Cu") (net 5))
 (segment (start 182.087994 73.66) (end 186.532994 78.105) (width 0.6) (layer "B.Cu") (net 5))
 (segment (start 137.03 62.36) (end 152.475 62.36) (width 0.6) (layer "B.Cu") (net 5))
 (segment (start 170.815 74.93) (end 169.545 73.66) (width 0.6) (layer "B.Cu") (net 5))
 (segment (start 112.3975 88.9025) (end 112.3975 71.785) (width 1.2) (layer "B.Cu") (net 5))
 (segment (start 162.56 73.66) (end 161.29 72.39) (width 0.6) (layer "B.Cu") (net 5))
 (segment (start 172.085 73.66) (end 182.087994 73.66) (width 0.6) (layer "B.Cu") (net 5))
 (segment (start 126.365 89.535) (end 130.81 93.98) (width 0.6) (layer "B.Cu") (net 5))
 (segment (start 186.532994 78.105) (end 187.325 78.105) (width 0.6) (layer "B.Cu") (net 5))
 (segment (start 166.37 71.12) (end 168.37 69.12) (width 0.6) (layer "B.Cu") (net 5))
 (segment (start 127.605 71.785) (end 137.03 62.36) (width 0.6) (layer "B.Cu") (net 5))
 (segment (start 161.29 72.39) (end 161.29 64.135) (width 0.6) (layer "B.Cu") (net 5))
 (segment (start 166.37 73.66) (end 162.56 73.66) (width 0.6) (layer "B.Cu") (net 5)))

